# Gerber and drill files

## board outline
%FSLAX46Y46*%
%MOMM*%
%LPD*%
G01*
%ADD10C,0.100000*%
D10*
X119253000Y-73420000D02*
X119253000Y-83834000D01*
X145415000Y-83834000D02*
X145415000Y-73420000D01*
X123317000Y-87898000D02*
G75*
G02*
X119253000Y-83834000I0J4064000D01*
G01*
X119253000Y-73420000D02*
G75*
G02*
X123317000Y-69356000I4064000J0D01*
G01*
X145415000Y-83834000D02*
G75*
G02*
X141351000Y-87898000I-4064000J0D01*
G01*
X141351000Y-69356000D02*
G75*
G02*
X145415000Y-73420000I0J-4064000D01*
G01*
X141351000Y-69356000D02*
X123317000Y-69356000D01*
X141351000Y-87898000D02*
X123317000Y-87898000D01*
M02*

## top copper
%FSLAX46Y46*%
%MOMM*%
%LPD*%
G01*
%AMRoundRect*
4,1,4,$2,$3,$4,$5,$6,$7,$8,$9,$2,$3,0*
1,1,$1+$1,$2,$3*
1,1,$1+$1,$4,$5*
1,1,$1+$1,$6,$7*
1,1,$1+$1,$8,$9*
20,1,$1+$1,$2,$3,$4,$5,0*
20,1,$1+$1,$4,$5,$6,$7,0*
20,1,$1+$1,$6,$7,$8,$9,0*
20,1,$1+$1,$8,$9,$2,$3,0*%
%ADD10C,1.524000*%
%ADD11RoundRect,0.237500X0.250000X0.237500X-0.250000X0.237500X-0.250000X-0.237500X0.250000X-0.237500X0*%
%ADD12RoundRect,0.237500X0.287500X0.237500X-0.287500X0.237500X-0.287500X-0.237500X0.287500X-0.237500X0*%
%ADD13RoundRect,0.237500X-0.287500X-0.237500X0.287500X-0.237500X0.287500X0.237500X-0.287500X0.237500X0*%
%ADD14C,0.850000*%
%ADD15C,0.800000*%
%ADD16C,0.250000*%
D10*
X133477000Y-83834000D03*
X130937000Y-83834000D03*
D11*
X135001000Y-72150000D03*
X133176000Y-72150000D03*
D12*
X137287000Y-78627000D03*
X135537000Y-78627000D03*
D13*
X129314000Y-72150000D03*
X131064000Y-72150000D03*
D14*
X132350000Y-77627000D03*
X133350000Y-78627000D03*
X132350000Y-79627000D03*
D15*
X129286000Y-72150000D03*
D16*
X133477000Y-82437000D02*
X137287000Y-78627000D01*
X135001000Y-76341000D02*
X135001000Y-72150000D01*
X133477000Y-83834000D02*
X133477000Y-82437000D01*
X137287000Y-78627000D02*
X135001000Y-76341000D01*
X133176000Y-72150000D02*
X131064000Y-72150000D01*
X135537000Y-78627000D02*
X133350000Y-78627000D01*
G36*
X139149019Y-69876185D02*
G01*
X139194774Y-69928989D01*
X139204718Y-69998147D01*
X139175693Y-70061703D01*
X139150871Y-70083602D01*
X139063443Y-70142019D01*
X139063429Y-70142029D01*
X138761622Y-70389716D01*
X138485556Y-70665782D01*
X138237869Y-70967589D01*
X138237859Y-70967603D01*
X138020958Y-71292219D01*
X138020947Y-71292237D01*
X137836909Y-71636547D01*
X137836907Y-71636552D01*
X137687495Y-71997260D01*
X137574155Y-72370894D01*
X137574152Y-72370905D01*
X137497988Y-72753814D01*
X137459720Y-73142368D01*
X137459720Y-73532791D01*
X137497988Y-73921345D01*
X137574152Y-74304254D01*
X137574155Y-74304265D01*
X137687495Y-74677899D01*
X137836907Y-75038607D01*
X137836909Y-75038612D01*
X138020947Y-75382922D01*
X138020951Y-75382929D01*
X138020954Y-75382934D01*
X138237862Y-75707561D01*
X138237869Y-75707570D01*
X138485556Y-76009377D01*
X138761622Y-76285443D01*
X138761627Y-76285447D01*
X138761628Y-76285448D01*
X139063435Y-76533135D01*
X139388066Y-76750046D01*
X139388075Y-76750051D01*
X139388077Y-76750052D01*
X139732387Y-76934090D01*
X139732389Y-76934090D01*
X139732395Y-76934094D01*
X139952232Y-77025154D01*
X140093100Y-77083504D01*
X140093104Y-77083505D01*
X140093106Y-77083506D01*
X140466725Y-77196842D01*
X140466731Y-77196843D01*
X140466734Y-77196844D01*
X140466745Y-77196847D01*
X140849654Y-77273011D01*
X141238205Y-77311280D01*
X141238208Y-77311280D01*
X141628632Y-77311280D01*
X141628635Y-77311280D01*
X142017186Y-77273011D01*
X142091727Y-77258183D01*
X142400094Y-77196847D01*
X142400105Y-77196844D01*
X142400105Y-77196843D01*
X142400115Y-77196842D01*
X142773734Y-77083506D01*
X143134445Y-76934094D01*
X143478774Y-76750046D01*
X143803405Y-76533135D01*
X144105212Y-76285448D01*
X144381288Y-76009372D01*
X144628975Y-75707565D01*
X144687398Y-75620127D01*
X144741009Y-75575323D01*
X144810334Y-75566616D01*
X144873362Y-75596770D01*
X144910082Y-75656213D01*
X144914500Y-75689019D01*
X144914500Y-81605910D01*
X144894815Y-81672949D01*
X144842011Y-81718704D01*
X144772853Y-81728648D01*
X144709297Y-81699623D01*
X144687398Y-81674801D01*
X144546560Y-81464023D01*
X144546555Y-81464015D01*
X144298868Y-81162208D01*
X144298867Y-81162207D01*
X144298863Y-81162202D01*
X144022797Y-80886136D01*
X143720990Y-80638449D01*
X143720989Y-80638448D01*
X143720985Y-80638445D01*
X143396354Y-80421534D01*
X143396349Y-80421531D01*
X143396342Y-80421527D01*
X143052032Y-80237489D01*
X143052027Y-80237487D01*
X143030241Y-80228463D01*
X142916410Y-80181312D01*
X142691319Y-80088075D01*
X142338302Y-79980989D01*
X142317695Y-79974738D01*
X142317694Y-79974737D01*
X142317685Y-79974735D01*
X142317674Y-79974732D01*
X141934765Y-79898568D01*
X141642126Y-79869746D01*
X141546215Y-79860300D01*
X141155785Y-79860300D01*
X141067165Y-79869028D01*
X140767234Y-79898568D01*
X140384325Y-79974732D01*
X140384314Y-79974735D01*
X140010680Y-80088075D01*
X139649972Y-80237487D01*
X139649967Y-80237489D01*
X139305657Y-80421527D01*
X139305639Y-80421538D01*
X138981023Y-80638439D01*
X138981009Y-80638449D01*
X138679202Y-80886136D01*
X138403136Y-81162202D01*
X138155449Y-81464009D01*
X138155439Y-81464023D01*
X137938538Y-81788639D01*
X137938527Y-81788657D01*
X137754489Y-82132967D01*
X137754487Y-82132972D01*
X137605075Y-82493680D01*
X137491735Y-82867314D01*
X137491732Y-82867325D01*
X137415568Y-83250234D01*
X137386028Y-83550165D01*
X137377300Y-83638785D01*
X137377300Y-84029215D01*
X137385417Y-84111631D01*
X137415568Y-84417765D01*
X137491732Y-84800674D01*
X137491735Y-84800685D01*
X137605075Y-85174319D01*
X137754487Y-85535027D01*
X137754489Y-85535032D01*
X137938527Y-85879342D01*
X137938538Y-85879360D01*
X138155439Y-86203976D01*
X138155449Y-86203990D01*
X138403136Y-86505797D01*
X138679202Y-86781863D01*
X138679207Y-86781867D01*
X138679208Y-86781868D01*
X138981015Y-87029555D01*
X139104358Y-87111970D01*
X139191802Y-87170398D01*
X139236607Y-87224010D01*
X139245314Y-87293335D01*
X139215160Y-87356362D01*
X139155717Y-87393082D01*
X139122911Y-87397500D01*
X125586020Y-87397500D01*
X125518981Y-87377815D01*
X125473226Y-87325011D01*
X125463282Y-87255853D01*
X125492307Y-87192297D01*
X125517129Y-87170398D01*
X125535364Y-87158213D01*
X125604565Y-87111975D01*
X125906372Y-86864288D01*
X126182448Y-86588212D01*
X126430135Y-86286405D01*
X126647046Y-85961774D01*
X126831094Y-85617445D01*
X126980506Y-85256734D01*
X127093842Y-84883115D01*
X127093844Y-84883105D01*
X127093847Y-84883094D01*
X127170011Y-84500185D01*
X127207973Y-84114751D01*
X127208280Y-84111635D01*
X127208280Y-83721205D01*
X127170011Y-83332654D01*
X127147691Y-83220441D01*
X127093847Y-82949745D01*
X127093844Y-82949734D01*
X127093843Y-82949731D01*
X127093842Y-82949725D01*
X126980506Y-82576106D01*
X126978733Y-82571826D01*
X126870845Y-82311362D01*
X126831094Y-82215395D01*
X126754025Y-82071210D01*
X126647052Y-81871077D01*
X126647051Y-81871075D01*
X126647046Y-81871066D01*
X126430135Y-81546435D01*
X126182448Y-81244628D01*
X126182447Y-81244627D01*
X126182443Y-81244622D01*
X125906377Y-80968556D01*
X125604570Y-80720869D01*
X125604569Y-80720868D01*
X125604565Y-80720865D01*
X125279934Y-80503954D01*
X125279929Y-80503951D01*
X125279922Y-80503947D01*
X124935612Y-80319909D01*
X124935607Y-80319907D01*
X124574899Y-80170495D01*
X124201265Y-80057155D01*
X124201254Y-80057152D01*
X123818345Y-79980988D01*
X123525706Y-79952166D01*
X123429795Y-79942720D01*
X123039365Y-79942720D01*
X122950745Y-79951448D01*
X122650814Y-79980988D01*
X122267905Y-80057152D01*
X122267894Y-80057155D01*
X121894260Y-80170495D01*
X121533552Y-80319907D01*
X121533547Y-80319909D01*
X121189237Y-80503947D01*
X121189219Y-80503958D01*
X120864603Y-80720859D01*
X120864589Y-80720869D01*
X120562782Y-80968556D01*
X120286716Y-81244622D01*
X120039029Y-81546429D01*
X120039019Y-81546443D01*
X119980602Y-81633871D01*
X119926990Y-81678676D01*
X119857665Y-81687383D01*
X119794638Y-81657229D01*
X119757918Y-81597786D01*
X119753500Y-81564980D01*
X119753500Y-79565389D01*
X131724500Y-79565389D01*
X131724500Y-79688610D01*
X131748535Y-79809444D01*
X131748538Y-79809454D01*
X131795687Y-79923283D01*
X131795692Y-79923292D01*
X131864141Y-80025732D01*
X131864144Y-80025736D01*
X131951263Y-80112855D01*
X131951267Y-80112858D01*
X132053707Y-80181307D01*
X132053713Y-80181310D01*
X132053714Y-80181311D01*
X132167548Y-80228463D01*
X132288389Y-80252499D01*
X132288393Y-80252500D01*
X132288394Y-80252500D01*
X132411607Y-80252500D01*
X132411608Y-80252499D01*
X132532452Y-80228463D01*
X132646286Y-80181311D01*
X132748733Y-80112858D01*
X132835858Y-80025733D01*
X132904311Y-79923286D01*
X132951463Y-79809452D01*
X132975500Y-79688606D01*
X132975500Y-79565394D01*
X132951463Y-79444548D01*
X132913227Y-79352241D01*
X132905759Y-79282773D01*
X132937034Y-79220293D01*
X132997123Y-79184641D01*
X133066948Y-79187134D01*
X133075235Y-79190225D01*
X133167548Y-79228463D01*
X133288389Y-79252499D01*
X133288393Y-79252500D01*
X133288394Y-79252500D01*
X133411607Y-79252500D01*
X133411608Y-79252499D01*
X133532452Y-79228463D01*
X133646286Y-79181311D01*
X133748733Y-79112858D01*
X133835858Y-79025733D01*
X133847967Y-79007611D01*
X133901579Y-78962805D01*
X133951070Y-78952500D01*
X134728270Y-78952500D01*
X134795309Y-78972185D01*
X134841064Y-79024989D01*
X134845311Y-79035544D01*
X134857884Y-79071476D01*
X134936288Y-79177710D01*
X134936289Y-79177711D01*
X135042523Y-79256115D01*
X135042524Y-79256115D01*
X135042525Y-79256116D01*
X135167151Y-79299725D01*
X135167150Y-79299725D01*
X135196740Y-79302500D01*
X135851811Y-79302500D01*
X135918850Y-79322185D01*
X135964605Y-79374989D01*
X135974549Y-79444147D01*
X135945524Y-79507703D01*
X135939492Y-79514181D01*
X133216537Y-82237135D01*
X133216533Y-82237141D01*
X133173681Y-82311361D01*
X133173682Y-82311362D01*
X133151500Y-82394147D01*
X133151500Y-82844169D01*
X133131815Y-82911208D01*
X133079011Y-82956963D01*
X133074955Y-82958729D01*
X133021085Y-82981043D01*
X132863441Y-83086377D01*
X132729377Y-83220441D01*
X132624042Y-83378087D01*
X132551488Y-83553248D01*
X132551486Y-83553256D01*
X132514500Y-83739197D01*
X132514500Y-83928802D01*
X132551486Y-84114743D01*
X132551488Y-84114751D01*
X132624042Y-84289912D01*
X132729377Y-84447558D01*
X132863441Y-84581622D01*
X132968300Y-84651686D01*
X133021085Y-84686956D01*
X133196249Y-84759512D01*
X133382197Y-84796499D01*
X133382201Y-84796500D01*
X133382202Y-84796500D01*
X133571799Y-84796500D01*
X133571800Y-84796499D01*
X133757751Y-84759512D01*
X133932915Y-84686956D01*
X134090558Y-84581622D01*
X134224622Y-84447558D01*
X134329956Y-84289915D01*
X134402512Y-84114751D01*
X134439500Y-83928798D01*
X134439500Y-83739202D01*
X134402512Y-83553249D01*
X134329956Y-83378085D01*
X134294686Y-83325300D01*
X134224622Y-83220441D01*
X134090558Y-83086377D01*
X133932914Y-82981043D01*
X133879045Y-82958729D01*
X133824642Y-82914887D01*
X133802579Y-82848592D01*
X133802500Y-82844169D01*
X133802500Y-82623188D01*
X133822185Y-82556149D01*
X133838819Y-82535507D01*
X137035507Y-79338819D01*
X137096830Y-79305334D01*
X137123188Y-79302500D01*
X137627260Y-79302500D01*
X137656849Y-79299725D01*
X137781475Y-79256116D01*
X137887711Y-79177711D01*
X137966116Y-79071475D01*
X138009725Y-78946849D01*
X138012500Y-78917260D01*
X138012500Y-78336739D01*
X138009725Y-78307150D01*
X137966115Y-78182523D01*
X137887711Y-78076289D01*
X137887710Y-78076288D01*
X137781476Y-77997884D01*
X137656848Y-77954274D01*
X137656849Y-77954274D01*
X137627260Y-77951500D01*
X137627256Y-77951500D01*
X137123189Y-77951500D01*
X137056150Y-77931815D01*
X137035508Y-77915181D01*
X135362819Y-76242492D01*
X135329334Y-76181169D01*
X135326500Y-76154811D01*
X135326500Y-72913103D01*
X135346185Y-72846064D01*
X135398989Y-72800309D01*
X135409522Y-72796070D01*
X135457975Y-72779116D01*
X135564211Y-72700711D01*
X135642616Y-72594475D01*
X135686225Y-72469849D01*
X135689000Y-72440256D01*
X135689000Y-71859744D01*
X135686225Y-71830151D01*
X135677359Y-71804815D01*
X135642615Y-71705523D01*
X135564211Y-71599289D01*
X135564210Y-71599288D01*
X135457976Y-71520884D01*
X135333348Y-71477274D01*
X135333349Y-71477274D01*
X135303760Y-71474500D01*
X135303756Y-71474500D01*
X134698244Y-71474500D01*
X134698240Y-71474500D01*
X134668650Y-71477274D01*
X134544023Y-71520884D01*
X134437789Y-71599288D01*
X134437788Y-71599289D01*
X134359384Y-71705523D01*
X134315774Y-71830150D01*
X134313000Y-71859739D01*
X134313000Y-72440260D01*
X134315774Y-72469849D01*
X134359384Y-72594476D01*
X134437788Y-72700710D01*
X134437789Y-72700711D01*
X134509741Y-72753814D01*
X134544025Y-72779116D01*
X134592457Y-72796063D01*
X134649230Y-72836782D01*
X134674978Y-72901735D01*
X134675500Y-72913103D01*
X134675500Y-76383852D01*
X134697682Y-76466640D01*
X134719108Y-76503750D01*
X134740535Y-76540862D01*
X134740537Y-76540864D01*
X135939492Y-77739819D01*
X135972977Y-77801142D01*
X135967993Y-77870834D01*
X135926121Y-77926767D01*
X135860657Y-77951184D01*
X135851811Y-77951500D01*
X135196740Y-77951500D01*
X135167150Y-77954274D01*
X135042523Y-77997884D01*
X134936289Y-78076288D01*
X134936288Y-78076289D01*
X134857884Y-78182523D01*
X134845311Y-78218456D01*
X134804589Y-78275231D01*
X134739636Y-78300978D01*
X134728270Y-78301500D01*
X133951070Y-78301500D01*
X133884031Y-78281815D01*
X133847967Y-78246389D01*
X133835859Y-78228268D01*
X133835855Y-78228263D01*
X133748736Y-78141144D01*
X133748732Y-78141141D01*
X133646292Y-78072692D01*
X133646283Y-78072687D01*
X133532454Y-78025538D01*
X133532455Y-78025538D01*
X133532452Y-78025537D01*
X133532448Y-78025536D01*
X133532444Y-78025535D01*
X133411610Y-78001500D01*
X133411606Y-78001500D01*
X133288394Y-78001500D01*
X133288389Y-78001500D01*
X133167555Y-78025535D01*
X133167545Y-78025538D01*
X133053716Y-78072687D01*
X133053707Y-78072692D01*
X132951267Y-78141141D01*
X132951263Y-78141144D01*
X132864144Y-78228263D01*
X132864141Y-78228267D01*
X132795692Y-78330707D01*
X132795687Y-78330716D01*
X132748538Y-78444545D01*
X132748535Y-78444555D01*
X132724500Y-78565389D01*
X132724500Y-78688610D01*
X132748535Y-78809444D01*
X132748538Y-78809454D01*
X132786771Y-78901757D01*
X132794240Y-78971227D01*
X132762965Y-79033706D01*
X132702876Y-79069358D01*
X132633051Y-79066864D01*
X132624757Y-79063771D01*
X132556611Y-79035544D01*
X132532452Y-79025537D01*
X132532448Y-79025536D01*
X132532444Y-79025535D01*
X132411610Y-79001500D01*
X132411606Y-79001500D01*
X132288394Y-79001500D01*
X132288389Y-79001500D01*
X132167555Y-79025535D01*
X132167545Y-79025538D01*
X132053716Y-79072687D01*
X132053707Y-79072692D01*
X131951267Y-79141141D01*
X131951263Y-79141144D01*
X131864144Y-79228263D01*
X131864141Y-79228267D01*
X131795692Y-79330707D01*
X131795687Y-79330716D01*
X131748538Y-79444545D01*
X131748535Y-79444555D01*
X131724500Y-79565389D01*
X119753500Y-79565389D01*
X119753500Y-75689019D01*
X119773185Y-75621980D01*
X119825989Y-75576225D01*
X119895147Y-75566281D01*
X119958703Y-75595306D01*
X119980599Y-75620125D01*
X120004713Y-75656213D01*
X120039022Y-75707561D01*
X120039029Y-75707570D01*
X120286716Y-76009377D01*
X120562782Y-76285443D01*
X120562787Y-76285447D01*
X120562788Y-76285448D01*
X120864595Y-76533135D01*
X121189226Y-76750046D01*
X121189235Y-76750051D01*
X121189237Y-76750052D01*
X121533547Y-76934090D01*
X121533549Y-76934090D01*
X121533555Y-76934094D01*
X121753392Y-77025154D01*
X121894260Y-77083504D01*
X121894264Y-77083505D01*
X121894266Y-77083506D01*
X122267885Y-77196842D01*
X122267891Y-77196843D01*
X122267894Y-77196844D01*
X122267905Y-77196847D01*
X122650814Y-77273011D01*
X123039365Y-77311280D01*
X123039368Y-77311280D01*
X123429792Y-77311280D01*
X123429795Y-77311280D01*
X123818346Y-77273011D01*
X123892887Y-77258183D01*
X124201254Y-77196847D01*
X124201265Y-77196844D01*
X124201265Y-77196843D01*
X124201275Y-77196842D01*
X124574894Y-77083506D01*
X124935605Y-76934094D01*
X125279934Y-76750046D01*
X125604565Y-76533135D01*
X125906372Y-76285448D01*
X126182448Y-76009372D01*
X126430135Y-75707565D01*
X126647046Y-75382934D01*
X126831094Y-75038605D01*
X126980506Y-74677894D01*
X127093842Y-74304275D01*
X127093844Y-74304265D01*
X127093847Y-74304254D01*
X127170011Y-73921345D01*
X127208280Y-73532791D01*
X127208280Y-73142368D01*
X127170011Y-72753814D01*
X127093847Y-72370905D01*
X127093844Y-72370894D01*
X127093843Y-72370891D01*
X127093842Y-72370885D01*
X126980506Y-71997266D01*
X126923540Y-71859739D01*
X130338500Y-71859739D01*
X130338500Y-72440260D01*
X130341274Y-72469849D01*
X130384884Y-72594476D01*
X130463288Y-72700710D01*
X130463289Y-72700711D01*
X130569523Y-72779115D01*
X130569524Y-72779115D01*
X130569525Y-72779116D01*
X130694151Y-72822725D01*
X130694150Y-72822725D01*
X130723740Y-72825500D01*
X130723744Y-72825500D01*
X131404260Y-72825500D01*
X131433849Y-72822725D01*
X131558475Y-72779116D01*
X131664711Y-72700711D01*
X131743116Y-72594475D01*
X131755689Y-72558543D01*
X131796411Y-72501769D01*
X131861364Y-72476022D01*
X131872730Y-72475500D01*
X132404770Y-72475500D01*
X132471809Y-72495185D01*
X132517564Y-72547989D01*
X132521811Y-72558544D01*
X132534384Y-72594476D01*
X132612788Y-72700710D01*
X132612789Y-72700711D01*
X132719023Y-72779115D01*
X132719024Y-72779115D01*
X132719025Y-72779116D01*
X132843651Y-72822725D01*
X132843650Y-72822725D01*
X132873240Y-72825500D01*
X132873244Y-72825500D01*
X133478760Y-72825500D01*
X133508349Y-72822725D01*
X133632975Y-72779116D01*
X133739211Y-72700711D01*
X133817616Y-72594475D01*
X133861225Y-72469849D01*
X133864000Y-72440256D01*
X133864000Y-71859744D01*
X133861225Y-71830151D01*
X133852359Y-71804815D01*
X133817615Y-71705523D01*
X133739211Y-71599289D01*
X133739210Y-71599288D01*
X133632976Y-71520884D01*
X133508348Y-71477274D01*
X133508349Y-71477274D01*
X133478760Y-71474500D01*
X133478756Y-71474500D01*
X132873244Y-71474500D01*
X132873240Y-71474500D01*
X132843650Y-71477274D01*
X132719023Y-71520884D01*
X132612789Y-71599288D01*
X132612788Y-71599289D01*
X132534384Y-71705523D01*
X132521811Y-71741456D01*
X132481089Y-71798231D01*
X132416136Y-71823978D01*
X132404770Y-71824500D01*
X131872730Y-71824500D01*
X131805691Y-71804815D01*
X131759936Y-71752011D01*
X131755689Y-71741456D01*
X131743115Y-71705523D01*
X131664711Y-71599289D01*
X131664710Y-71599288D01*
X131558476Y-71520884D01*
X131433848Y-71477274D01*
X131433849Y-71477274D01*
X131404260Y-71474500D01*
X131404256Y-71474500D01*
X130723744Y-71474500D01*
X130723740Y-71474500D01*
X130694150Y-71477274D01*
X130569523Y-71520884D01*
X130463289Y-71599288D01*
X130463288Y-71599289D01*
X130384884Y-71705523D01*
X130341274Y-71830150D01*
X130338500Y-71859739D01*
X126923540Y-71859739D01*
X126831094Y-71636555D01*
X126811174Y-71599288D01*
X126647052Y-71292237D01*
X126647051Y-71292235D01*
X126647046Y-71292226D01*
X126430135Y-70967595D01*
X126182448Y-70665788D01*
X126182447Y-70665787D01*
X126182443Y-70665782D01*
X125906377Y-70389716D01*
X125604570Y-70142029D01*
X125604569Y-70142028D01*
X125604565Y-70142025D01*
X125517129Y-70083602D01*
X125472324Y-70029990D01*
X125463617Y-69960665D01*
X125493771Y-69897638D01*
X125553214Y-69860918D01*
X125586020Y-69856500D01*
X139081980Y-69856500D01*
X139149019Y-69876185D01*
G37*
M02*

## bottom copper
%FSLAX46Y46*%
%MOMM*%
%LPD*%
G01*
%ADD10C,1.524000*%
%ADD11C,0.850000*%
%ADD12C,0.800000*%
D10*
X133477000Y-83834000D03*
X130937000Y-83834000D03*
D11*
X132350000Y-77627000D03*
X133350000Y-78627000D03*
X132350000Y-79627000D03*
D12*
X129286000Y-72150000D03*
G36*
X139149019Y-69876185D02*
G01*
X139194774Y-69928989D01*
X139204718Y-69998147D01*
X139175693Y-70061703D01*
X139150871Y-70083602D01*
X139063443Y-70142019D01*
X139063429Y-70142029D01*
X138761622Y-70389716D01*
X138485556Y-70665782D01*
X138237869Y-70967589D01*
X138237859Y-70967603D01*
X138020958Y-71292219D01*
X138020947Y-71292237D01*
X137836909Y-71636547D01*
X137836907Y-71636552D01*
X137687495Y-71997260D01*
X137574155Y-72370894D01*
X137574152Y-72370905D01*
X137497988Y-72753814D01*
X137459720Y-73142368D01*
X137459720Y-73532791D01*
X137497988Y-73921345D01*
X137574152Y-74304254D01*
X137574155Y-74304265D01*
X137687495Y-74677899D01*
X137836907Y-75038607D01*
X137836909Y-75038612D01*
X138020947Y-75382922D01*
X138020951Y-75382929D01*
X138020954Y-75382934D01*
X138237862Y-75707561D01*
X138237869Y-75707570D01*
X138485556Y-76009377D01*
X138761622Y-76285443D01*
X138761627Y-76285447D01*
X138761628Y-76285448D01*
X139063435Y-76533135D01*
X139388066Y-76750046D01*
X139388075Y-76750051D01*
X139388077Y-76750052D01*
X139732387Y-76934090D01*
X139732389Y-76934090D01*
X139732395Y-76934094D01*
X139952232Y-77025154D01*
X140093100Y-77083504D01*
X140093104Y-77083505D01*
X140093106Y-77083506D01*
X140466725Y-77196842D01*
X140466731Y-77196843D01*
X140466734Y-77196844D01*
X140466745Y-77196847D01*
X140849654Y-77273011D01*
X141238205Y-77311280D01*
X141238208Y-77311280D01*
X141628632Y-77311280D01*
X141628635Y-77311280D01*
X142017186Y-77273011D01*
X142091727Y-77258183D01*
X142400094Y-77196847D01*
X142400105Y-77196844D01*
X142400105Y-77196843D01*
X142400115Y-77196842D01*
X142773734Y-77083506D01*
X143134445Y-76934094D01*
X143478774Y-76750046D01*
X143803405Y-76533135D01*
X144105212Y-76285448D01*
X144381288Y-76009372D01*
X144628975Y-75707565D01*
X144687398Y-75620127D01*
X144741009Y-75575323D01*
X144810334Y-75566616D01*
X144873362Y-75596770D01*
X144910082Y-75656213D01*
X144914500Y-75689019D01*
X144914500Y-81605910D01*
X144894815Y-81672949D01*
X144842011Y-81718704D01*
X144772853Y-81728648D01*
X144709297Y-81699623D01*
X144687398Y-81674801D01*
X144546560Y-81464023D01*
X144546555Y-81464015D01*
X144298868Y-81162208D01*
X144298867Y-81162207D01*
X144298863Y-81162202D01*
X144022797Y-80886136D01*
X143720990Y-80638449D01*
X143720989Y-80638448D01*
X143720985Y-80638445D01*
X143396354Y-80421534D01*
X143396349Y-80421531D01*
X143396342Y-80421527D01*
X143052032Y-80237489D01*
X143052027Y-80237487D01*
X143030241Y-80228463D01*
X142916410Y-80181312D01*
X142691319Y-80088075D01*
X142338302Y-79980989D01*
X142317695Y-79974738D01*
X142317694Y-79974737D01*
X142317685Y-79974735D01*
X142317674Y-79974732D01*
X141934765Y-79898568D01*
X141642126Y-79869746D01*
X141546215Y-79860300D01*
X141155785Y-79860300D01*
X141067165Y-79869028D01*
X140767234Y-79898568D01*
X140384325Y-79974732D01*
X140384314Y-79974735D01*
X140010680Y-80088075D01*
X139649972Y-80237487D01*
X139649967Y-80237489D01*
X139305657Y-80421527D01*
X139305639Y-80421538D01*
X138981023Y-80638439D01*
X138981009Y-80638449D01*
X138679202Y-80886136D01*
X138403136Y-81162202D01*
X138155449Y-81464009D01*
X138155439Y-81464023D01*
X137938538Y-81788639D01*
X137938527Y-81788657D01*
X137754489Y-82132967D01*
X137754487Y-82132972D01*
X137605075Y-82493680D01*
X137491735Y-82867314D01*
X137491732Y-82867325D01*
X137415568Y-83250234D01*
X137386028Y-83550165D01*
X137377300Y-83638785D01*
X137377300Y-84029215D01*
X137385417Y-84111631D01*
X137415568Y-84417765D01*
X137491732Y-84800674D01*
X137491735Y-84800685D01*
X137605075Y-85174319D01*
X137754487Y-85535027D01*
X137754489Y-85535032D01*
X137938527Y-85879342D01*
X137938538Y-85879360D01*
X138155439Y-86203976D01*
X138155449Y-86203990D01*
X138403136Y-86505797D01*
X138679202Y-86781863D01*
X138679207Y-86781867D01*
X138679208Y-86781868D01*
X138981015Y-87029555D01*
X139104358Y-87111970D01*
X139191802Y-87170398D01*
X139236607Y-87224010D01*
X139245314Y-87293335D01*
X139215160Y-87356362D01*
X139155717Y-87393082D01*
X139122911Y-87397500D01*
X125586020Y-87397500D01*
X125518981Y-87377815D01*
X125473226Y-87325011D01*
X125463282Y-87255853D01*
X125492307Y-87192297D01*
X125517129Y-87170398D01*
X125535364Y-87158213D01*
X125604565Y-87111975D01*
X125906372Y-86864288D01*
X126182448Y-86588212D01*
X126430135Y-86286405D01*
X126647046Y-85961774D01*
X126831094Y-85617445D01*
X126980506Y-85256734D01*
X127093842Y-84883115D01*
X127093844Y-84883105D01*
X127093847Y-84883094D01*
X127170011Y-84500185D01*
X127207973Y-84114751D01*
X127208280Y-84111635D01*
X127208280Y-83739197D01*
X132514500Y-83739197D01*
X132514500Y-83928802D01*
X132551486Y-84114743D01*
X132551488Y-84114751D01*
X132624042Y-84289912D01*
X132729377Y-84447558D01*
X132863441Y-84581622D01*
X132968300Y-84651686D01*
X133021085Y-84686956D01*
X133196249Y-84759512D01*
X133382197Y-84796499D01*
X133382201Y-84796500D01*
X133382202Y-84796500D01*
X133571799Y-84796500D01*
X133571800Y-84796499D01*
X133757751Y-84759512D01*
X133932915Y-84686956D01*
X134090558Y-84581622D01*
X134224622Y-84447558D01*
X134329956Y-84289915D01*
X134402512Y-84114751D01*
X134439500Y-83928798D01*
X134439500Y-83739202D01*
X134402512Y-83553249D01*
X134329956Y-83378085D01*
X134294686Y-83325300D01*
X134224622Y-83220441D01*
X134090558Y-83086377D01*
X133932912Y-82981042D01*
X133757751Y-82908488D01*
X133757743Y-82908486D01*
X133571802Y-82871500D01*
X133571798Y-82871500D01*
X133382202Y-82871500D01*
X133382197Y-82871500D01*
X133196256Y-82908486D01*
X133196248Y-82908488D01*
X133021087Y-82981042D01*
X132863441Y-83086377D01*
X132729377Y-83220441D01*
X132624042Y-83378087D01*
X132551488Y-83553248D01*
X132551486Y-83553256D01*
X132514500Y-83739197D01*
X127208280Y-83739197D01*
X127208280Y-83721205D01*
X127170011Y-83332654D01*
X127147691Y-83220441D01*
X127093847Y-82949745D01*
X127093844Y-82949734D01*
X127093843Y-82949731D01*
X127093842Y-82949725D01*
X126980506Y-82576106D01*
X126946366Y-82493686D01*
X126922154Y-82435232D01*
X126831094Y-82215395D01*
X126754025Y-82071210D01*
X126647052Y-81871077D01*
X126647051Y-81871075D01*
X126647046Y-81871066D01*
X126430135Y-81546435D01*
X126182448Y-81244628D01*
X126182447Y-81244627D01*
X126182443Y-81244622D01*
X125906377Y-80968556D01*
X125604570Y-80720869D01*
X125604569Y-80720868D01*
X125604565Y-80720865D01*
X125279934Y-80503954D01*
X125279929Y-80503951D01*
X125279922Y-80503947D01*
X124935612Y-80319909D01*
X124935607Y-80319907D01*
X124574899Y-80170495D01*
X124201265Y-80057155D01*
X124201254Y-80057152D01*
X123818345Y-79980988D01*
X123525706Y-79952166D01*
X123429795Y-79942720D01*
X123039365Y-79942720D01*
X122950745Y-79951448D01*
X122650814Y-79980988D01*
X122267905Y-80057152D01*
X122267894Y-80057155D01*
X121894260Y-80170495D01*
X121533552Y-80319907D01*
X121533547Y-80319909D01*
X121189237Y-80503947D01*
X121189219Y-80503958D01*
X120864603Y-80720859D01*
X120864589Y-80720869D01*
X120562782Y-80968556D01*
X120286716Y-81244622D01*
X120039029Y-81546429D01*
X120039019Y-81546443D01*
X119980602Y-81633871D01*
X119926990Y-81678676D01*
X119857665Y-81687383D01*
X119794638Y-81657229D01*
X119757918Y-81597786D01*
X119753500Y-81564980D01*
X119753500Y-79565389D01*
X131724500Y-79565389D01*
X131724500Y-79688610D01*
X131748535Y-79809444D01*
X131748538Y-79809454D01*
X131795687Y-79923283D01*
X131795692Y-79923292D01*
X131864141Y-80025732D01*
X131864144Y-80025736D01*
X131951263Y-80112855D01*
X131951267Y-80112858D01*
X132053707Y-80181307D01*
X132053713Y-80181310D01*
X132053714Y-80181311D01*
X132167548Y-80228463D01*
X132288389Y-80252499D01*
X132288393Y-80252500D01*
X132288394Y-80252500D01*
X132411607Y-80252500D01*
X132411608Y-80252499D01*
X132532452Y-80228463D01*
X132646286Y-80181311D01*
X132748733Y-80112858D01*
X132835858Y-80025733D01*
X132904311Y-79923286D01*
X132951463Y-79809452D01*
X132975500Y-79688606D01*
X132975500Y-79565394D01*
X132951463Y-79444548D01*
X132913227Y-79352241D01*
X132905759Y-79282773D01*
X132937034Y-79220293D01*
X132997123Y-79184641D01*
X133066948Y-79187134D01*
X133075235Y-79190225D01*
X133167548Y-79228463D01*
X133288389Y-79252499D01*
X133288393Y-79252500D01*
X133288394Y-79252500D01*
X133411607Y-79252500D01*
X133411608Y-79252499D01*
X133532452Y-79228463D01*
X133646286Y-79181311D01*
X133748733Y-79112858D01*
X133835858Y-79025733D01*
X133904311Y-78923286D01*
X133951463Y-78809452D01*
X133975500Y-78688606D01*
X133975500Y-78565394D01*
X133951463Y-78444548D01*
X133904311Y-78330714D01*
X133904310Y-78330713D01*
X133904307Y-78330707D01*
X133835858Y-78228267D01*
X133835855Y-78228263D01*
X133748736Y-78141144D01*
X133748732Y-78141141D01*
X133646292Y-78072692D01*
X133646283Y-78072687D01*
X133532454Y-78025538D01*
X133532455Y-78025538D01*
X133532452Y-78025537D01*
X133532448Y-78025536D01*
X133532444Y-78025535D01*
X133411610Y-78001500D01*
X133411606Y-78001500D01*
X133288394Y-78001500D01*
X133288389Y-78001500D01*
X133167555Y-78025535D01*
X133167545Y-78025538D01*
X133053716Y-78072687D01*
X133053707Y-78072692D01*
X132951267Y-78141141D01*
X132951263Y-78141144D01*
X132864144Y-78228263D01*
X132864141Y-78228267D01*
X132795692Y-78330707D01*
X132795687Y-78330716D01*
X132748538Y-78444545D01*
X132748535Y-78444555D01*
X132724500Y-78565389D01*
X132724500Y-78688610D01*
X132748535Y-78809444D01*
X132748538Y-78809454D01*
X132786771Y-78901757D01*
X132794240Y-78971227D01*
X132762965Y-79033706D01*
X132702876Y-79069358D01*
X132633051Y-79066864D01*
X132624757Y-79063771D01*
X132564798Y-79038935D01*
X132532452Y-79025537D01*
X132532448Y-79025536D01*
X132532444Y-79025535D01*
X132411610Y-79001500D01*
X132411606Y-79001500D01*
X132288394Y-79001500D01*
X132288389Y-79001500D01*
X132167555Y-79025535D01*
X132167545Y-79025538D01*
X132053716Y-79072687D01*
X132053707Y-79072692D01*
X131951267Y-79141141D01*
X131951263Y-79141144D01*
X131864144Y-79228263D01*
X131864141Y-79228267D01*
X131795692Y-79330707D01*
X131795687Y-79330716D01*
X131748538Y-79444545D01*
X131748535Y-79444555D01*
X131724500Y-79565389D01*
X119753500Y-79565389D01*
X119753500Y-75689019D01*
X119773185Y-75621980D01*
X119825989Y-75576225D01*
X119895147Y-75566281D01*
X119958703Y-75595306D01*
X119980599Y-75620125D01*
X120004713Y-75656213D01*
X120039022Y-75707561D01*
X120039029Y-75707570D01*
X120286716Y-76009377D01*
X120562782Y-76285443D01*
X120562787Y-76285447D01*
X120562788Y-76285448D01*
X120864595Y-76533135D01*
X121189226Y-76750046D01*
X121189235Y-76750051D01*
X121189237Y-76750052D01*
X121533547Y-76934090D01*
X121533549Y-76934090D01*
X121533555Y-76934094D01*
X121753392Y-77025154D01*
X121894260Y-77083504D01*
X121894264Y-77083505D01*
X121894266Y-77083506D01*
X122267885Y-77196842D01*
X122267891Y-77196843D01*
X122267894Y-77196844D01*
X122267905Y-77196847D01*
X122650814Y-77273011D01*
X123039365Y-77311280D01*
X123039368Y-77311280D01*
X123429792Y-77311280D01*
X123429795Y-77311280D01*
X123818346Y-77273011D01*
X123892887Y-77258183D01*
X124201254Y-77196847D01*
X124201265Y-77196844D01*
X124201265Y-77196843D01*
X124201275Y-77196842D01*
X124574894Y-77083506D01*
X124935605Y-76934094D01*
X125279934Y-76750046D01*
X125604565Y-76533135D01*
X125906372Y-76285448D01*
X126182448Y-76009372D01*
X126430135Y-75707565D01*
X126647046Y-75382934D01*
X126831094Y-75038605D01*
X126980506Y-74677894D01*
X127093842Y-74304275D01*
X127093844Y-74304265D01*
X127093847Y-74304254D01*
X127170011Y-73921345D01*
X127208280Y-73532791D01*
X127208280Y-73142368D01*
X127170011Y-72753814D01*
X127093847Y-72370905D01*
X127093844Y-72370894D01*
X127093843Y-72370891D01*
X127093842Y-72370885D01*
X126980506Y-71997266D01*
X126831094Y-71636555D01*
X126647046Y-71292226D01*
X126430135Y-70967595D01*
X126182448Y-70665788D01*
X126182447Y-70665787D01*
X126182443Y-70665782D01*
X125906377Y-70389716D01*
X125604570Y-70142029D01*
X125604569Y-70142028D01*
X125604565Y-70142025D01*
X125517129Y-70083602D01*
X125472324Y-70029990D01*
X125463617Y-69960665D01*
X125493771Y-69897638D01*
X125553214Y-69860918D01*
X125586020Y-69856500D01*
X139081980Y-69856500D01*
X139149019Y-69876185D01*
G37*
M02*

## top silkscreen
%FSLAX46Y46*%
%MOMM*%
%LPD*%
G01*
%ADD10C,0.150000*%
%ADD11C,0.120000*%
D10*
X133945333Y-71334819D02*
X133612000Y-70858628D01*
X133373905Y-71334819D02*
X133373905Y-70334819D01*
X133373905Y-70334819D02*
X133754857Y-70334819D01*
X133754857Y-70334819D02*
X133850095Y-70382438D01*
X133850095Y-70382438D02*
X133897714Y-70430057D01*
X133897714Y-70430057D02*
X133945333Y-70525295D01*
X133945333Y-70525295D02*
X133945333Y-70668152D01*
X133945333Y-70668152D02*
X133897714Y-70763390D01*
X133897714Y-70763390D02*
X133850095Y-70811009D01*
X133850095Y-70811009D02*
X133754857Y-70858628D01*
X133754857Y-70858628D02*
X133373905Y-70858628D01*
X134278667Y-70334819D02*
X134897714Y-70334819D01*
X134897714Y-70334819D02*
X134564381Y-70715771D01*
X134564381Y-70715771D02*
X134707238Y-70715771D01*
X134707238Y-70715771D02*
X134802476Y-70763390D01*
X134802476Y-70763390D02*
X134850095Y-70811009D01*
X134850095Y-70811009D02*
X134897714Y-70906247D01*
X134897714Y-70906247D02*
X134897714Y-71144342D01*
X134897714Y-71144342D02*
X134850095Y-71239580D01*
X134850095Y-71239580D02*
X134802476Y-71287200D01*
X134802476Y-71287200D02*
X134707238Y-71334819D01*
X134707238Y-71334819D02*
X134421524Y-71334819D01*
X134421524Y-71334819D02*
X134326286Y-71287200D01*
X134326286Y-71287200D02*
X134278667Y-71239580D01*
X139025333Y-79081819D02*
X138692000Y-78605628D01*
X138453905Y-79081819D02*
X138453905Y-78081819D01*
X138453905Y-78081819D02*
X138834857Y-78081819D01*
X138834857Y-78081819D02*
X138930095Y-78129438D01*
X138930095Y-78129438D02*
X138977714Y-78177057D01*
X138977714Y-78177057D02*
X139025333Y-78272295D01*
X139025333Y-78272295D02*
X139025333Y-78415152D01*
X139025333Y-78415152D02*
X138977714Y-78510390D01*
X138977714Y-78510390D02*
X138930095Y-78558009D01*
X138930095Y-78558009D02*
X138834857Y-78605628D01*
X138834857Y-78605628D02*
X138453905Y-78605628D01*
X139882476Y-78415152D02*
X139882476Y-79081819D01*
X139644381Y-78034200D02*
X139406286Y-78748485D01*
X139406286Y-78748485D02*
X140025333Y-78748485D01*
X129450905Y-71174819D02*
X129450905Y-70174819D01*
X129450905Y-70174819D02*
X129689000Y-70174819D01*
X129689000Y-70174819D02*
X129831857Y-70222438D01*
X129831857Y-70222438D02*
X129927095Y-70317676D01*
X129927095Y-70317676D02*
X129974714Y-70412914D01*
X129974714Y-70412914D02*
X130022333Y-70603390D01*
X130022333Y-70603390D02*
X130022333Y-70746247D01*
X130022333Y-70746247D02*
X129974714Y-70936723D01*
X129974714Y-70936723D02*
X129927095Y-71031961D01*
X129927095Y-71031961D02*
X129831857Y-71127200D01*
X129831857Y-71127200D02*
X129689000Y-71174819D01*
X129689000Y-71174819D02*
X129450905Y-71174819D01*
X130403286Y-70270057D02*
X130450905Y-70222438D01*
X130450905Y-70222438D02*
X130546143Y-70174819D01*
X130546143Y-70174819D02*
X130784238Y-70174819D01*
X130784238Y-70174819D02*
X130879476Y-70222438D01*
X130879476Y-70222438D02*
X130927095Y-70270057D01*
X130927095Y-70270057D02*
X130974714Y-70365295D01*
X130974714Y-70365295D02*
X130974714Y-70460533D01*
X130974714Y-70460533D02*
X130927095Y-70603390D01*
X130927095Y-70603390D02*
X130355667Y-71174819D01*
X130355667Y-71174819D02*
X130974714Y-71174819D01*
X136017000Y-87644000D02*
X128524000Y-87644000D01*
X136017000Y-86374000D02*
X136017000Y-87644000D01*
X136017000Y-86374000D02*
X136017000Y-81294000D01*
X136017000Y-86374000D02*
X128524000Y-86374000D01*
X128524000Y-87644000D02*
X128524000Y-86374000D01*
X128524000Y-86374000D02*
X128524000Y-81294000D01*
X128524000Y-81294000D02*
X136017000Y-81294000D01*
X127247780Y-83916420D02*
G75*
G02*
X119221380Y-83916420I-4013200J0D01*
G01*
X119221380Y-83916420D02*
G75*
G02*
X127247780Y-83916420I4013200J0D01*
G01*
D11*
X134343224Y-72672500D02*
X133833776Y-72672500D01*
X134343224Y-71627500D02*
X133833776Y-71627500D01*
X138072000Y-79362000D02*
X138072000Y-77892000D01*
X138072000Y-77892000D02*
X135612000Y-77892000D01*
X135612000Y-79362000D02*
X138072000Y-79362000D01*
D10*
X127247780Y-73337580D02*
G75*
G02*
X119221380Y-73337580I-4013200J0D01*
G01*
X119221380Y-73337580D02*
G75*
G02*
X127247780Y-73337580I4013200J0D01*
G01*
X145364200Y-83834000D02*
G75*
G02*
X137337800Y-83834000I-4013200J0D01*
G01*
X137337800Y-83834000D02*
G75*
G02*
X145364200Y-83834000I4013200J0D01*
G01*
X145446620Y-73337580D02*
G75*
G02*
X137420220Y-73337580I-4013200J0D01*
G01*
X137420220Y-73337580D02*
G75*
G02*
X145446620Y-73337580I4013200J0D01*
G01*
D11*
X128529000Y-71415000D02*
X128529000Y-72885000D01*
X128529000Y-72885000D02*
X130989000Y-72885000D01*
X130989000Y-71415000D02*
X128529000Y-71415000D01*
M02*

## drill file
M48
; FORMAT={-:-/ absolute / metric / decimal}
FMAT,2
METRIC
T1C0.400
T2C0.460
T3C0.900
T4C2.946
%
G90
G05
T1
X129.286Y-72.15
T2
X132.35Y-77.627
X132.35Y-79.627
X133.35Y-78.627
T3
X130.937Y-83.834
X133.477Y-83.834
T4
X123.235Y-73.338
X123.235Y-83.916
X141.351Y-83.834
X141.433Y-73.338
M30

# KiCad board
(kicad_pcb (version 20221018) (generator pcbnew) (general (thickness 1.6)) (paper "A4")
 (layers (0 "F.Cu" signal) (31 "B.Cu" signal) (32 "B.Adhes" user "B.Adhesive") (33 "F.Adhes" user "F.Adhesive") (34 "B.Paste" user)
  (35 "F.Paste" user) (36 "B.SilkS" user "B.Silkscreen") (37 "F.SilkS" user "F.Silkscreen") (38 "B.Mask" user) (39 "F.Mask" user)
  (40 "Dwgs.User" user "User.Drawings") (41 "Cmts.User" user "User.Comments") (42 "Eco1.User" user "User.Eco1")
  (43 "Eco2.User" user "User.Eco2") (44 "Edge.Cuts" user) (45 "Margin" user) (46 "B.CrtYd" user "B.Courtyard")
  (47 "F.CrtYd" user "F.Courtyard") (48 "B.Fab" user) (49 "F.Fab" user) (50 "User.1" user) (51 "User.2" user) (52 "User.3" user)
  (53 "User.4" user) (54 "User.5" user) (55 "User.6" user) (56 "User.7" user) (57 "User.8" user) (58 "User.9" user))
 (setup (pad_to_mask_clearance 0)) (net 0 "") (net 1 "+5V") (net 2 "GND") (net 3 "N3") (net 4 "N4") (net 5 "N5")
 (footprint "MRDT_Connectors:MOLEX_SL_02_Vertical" (layer "F.Cu") (at 133.477 83.834 180)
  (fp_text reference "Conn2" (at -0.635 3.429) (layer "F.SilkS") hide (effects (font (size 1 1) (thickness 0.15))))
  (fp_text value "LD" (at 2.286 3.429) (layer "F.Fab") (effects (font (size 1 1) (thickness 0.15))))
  (fp_line (start -2.54 -3.81) (end 4.953 -3.81) (stroke (width 0.15) (type solid)) (layer "F.SilkS"))
  (fp_line (start -2.54 -2.54) (end -2.54 -3.81) (stroke (width 0.15) (type solid)) (layer "F.SilkS"))
  (fp_line (start -2.54 -2.54) (end -2.54 2.54) (stroke (width 0.15) (type solid)) (layer "F.SilkS"))
  (fp_line (start -2.54 -2.54) (end 4.953 -2.54) (stroke (width 0.15) (type solid)) (layer "F.SilkS"))
  (fp_line (start 4.953 -3.81) (end 4.953 -2.54) (stroke (width 0.15) (type solid)) (layer "F.SilkS"))
  (fp_line (start 4.953 -2.54) (end 4.953 2.54) (stroke (width 0.15) (type solid)) (layer "F.SilkS"))
  (fp_line (start 4.953 2.54) (end -2.54 2.54) (stroke (width 0.15) (type solid)) (layer "F.SilkS"))
  (pad "1" thru_hole circle (at 0 0 180) (size 1.524 1.524) (drill 0.9) (layers "*.Cu" "*.Mask") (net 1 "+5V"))
  (pad "2" thru_hole circle (at 2.54 0 180) (size 1.524 1.524) (drill 0.9) (layers "*.Cu" "*.Mask") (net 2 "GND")))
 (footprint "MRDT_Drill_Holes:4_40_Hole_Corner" (layer "F.Cu") (at 127.2427 79.9083 180)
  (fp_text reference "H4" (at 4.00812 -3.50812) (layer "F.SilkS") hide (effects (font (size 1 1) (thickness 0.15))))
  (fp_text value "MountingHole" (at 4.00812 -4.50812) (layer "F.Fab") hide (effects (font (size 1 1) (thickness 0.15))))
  (fp_circle (center 4.00812 -4.00812) (end 4.00812 0.00508) (stroke (width 0.15) (type solid)) (fill none) (layer "F.SilkS"))
  (pad "" np_thru_hole circle (at 4.00812 -4.00812 180) (size 2.9464 2.9464) (drill 2.9464) (layers "*.Cu" "*.Mask") (clearance 2.5)))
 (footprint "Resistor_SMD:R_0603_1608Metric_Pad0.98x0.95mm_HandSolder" (layer "F.Cu") (at 134.0885 72.15 180)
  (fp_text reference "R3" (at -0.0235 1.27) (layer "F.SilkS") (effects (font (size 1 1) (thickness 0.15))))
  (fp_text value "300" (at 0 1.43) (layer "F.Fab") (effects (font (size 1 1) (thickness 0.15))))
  (fp_line (start -0.254724 -0.5225) (end 0.254724 -0.5225) (stroke (width 0.12) (type solid)) (layer "F.SilkS"))
  (fp_line (start -0.254724 0.5225) (end 0.254724 0.5225) (stroke (width 0.12) (type solid)) (layer "F.SilkS"))
  (pad "1" smd roundrect (at -0.9125 0 180) (size 0.975 0.95) (layers "F.Cu" "F.Paste" "F.Mask") (roundrect_rratio 0.25) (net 1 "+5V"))
  (pad "2" smd roundrect (at 0.9125 0 180) (size 0.975 0.95) (layers "F.Cu" "F.Paste" "F.Mask") (roundrect_rratio 0.25) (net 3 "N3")))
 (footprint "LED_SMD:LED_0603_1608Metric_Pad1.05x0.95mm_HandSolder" (layer "F.Cu") (at 136.412 78.627 180)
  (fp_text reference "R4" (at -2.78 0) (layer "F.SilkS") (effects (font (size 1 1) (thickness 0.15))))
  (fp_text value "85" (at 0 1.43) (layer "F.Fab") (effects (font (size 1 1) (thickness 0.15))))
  (fp_line (start -1.66 -0.735) (end -1.66 0.735) (stroke (width 0.12) (type solid)) (layer "F.SilkS"))
  (fp_line (start -1.66 0.735) (end 0.8 0.735) (stroke (width 0.12) (type solid)) (layer "F.SilkS"))
  (fp_line (start 0.8 -0.735) (end -1.66 -0.735) (stroke (width 0.12) (type solid)) (layer "F.SilkS"))
  (pad "1" smd roundrect (at -0.875 0 180) (size 1.05 0.95) (layers "F.Cu" "F.Paste" "F.Mask") (roundrect_rratio 0.25) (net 1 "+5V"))
  (pad "2" smd roundrect (at 0.875 0 180) (size 1.05 0.95) (layers "F.Cu" "F.Paste" "F.Mask") (roundrect_rratio 0.25) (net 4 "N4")))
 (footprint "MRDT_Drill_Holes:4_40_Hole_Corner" (layer "F.Cu") (at 127.2427 77.3457 90)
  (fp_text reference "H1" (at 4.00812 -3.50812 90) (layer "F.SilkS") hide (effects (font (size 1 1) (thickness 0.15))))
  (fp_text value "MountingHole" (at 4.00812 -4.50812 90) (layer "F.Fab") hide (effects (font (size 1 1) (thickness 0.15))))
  (fp_circle (center 4.00812 -4.00812) (end 4.00812 0.00508) (stroke (width 0.15) (type solid)) (fill none) (layer "F.SilkS"))
  (pad "" np_thru_hole circle (at 4.00812 -4.00812 90) (size 2.9464 2.9464) (drill 2.9464) (layers "*.Cu" "*.Mask") (clearance 2.5)))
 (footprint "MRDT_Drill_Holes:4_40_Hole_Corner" (layer "F.Cu") (at 137.34288 79.82588 -90)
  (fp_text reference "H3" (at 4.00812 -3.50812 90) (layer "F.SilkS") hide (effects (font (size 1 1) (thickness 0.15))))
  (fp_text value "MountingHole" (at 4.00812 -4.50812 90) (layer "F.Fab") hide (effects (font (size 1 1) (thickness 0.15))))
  (fp_circle (center 4.00812 -4.00812) (end 4.00812 0.00508) (stroke (width 0.15) (type solid)) (fill none) (layer "F.SilkS"))
  (pad "" np_thru_hole circle (at 4.00812 -4.00812 270) (size 2.9464 2.9464) (drill 2.9464) (layers "*.Cu" "*.Mask") (clearance 2.5)))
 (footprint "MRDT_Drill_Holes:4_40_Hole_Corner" (layer "F.Cu") (at 137.4253 77.3457)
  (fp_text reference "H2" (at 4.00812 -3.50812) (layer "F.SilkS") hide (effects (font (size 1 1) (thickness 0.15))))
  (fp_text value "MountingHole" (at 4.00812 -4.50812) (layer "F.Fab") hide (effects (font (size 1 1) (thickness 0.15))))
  (fp_circle (center 4.00812 -4.00812) (end 4.00812 0.00508) (stroke (width 0.15) (type solid)) (fill none) (layer "F.SilkS"))
  (pad "" np_thru_hole circle (at 4.00812 -4.00812) (size 2.9464 2.9464) (drill 2.9464) (layers "*.Cu" "*.Mask") (clearance 2.5)))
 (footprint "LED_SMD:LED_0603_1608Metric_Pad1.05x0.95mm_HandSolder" (layer "F.Cu") (at 130.189 72.15)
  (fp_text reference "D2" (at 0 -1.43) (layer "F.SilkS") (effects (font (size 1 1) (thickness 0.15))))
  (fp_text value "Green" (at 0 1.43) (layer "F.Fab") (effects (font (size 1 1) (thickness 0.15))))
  (fp_line (start -1.66 -0.735) (end -1.66 0.735) (stroke (width 0.12) (type solid)) (layer "F.SilkS"))
  (fp_line (start -1.66 0.735) (end 0.8 0.735) (stroke (width 0.12) (type solid)) (layer "F.SilkS"))
  (fp_line (start 0.8 -0.735) (end -1.66 -0.735) (stroke (width 0.12) (type solid)) (layer "F.SilkS"))
  (pad "1" smd roundrect (at -0.875 0) (size 1.05 0.95) (layers "F.Cu" "F.Paste" "F.Mask") (roundrect_rratio 0.25) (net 2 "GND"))
  (pad "2" smd roundrect (at 0.875 0) (size 1.05 0.95) (layers "F.Cu" "F.Paste" "F.Mask") (roundrect_rratio 0.25) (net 3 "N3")))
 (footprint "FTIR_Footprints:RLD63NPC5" (layer "B.Cu") (at 132.35 78.627 180)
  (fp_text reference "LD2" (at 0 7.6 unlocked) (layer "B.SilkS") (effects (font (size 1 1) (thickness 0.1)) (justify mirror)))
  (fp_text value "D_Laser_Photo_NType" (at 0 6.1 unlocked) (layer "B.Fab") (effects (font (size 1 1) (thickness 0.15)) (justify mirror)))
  (pad "1" thru_hole circle (at 0 1 180) (size 0.85 0.85) (drill 0.46) (layers "*.Cu" "*.Mask") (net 2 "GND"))
  (pad "2" thru_hole circle (at -1 0 180) (size 0.85 0.85) (drill 0.46) (layers "*.Cu" "*.Mask") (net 4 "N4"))
  (pad "3" thru_hole circle (at 0 -1 180) (size 0.85 0.85) (drill 0.46) (layers "*.Cu" "*.Mask") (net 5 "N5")))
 (gr_line (start 119.253 73.42) (end 119.253 83.834) (stroke (width 0.1) (type default)) (layer "Edge.Cuts"))
 (gr_line (start 145.415 83.834) (end 145.415 73.42) (stroke (width 0.1) (type default)) (layer "Edge.Cuts"))
 (gr_arc (start 123.317 87.898) (mid 120.443318 86.707682) (end 119.253 83.834) (stroke (width 0.1) (type default)) (layer "Edge.Cuts"))
 (gr_arc (start 119.253 73.42) (mid 120.443318 70.546318) (end 123.317 69.356) (stroke (width 0.1) (type default)) (layer "Edge.Cuts"))
 (gr_arc (start 145.415 83.834) (mid 144.224682 86.707682) (end 141.351 87.898) (stroke (width 0.1) (type default)) (layer "Edge.Cuts"))
 (gr_arc (start 141.351 69.356) (mid 144.224682 70.546318) (end 145.415 73.42) (stroke (width 0.1) (type default)) (layer "Edge.Cuts"))
 (gr_line (start 141.351 69.356) (end 123.317 69.356) (stroke (width 0.1) (type default)) (layer "Edge.Cuts"))
 (gr_line (start 141.351 87.898) (end 123.317 87.898) (stroke (width 0.1) (type default)) (layer "Edge.Cuts"))
 (segment (start 133.477 82.437) (end 137.287 78.627) (width 0.25) (layer "F.Cu") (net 1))
 (segment (start 135.001 76.341) (end 135.001 72.15) (width 0.25) (layer "F.Cu") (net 1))
 (segment (start 133.477 83.834) (end 133.477 82.437) (width 0.25) (layer "F.Cu") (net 1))
 (segment (start 137.287 78.627) (end 135.001 76.341) (width 0.25) (layer "F.Cu") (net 1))
 (via (at 129.286 72.15) (size 0.8) (drill 0.4) (layers "F.Cu" "B.Cu") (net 2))
 (segment (start 133.176 72.15) (end 131.064 72.15) (width 0.25) (layer "F.Cu") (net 3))
 (segment (start 135.537 78.627) (end 133.35 78.627) (width 0.25) (layer "F.Cu") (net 4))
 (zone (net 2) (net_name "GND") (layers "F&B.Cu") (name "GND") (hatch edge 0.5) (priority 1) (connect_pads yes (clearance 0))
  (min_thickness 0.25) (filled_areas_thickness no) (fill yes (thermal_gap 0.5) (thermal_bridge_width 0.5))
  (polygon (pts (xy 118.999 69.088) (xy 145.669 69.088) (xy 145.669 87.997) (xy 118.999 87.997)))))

